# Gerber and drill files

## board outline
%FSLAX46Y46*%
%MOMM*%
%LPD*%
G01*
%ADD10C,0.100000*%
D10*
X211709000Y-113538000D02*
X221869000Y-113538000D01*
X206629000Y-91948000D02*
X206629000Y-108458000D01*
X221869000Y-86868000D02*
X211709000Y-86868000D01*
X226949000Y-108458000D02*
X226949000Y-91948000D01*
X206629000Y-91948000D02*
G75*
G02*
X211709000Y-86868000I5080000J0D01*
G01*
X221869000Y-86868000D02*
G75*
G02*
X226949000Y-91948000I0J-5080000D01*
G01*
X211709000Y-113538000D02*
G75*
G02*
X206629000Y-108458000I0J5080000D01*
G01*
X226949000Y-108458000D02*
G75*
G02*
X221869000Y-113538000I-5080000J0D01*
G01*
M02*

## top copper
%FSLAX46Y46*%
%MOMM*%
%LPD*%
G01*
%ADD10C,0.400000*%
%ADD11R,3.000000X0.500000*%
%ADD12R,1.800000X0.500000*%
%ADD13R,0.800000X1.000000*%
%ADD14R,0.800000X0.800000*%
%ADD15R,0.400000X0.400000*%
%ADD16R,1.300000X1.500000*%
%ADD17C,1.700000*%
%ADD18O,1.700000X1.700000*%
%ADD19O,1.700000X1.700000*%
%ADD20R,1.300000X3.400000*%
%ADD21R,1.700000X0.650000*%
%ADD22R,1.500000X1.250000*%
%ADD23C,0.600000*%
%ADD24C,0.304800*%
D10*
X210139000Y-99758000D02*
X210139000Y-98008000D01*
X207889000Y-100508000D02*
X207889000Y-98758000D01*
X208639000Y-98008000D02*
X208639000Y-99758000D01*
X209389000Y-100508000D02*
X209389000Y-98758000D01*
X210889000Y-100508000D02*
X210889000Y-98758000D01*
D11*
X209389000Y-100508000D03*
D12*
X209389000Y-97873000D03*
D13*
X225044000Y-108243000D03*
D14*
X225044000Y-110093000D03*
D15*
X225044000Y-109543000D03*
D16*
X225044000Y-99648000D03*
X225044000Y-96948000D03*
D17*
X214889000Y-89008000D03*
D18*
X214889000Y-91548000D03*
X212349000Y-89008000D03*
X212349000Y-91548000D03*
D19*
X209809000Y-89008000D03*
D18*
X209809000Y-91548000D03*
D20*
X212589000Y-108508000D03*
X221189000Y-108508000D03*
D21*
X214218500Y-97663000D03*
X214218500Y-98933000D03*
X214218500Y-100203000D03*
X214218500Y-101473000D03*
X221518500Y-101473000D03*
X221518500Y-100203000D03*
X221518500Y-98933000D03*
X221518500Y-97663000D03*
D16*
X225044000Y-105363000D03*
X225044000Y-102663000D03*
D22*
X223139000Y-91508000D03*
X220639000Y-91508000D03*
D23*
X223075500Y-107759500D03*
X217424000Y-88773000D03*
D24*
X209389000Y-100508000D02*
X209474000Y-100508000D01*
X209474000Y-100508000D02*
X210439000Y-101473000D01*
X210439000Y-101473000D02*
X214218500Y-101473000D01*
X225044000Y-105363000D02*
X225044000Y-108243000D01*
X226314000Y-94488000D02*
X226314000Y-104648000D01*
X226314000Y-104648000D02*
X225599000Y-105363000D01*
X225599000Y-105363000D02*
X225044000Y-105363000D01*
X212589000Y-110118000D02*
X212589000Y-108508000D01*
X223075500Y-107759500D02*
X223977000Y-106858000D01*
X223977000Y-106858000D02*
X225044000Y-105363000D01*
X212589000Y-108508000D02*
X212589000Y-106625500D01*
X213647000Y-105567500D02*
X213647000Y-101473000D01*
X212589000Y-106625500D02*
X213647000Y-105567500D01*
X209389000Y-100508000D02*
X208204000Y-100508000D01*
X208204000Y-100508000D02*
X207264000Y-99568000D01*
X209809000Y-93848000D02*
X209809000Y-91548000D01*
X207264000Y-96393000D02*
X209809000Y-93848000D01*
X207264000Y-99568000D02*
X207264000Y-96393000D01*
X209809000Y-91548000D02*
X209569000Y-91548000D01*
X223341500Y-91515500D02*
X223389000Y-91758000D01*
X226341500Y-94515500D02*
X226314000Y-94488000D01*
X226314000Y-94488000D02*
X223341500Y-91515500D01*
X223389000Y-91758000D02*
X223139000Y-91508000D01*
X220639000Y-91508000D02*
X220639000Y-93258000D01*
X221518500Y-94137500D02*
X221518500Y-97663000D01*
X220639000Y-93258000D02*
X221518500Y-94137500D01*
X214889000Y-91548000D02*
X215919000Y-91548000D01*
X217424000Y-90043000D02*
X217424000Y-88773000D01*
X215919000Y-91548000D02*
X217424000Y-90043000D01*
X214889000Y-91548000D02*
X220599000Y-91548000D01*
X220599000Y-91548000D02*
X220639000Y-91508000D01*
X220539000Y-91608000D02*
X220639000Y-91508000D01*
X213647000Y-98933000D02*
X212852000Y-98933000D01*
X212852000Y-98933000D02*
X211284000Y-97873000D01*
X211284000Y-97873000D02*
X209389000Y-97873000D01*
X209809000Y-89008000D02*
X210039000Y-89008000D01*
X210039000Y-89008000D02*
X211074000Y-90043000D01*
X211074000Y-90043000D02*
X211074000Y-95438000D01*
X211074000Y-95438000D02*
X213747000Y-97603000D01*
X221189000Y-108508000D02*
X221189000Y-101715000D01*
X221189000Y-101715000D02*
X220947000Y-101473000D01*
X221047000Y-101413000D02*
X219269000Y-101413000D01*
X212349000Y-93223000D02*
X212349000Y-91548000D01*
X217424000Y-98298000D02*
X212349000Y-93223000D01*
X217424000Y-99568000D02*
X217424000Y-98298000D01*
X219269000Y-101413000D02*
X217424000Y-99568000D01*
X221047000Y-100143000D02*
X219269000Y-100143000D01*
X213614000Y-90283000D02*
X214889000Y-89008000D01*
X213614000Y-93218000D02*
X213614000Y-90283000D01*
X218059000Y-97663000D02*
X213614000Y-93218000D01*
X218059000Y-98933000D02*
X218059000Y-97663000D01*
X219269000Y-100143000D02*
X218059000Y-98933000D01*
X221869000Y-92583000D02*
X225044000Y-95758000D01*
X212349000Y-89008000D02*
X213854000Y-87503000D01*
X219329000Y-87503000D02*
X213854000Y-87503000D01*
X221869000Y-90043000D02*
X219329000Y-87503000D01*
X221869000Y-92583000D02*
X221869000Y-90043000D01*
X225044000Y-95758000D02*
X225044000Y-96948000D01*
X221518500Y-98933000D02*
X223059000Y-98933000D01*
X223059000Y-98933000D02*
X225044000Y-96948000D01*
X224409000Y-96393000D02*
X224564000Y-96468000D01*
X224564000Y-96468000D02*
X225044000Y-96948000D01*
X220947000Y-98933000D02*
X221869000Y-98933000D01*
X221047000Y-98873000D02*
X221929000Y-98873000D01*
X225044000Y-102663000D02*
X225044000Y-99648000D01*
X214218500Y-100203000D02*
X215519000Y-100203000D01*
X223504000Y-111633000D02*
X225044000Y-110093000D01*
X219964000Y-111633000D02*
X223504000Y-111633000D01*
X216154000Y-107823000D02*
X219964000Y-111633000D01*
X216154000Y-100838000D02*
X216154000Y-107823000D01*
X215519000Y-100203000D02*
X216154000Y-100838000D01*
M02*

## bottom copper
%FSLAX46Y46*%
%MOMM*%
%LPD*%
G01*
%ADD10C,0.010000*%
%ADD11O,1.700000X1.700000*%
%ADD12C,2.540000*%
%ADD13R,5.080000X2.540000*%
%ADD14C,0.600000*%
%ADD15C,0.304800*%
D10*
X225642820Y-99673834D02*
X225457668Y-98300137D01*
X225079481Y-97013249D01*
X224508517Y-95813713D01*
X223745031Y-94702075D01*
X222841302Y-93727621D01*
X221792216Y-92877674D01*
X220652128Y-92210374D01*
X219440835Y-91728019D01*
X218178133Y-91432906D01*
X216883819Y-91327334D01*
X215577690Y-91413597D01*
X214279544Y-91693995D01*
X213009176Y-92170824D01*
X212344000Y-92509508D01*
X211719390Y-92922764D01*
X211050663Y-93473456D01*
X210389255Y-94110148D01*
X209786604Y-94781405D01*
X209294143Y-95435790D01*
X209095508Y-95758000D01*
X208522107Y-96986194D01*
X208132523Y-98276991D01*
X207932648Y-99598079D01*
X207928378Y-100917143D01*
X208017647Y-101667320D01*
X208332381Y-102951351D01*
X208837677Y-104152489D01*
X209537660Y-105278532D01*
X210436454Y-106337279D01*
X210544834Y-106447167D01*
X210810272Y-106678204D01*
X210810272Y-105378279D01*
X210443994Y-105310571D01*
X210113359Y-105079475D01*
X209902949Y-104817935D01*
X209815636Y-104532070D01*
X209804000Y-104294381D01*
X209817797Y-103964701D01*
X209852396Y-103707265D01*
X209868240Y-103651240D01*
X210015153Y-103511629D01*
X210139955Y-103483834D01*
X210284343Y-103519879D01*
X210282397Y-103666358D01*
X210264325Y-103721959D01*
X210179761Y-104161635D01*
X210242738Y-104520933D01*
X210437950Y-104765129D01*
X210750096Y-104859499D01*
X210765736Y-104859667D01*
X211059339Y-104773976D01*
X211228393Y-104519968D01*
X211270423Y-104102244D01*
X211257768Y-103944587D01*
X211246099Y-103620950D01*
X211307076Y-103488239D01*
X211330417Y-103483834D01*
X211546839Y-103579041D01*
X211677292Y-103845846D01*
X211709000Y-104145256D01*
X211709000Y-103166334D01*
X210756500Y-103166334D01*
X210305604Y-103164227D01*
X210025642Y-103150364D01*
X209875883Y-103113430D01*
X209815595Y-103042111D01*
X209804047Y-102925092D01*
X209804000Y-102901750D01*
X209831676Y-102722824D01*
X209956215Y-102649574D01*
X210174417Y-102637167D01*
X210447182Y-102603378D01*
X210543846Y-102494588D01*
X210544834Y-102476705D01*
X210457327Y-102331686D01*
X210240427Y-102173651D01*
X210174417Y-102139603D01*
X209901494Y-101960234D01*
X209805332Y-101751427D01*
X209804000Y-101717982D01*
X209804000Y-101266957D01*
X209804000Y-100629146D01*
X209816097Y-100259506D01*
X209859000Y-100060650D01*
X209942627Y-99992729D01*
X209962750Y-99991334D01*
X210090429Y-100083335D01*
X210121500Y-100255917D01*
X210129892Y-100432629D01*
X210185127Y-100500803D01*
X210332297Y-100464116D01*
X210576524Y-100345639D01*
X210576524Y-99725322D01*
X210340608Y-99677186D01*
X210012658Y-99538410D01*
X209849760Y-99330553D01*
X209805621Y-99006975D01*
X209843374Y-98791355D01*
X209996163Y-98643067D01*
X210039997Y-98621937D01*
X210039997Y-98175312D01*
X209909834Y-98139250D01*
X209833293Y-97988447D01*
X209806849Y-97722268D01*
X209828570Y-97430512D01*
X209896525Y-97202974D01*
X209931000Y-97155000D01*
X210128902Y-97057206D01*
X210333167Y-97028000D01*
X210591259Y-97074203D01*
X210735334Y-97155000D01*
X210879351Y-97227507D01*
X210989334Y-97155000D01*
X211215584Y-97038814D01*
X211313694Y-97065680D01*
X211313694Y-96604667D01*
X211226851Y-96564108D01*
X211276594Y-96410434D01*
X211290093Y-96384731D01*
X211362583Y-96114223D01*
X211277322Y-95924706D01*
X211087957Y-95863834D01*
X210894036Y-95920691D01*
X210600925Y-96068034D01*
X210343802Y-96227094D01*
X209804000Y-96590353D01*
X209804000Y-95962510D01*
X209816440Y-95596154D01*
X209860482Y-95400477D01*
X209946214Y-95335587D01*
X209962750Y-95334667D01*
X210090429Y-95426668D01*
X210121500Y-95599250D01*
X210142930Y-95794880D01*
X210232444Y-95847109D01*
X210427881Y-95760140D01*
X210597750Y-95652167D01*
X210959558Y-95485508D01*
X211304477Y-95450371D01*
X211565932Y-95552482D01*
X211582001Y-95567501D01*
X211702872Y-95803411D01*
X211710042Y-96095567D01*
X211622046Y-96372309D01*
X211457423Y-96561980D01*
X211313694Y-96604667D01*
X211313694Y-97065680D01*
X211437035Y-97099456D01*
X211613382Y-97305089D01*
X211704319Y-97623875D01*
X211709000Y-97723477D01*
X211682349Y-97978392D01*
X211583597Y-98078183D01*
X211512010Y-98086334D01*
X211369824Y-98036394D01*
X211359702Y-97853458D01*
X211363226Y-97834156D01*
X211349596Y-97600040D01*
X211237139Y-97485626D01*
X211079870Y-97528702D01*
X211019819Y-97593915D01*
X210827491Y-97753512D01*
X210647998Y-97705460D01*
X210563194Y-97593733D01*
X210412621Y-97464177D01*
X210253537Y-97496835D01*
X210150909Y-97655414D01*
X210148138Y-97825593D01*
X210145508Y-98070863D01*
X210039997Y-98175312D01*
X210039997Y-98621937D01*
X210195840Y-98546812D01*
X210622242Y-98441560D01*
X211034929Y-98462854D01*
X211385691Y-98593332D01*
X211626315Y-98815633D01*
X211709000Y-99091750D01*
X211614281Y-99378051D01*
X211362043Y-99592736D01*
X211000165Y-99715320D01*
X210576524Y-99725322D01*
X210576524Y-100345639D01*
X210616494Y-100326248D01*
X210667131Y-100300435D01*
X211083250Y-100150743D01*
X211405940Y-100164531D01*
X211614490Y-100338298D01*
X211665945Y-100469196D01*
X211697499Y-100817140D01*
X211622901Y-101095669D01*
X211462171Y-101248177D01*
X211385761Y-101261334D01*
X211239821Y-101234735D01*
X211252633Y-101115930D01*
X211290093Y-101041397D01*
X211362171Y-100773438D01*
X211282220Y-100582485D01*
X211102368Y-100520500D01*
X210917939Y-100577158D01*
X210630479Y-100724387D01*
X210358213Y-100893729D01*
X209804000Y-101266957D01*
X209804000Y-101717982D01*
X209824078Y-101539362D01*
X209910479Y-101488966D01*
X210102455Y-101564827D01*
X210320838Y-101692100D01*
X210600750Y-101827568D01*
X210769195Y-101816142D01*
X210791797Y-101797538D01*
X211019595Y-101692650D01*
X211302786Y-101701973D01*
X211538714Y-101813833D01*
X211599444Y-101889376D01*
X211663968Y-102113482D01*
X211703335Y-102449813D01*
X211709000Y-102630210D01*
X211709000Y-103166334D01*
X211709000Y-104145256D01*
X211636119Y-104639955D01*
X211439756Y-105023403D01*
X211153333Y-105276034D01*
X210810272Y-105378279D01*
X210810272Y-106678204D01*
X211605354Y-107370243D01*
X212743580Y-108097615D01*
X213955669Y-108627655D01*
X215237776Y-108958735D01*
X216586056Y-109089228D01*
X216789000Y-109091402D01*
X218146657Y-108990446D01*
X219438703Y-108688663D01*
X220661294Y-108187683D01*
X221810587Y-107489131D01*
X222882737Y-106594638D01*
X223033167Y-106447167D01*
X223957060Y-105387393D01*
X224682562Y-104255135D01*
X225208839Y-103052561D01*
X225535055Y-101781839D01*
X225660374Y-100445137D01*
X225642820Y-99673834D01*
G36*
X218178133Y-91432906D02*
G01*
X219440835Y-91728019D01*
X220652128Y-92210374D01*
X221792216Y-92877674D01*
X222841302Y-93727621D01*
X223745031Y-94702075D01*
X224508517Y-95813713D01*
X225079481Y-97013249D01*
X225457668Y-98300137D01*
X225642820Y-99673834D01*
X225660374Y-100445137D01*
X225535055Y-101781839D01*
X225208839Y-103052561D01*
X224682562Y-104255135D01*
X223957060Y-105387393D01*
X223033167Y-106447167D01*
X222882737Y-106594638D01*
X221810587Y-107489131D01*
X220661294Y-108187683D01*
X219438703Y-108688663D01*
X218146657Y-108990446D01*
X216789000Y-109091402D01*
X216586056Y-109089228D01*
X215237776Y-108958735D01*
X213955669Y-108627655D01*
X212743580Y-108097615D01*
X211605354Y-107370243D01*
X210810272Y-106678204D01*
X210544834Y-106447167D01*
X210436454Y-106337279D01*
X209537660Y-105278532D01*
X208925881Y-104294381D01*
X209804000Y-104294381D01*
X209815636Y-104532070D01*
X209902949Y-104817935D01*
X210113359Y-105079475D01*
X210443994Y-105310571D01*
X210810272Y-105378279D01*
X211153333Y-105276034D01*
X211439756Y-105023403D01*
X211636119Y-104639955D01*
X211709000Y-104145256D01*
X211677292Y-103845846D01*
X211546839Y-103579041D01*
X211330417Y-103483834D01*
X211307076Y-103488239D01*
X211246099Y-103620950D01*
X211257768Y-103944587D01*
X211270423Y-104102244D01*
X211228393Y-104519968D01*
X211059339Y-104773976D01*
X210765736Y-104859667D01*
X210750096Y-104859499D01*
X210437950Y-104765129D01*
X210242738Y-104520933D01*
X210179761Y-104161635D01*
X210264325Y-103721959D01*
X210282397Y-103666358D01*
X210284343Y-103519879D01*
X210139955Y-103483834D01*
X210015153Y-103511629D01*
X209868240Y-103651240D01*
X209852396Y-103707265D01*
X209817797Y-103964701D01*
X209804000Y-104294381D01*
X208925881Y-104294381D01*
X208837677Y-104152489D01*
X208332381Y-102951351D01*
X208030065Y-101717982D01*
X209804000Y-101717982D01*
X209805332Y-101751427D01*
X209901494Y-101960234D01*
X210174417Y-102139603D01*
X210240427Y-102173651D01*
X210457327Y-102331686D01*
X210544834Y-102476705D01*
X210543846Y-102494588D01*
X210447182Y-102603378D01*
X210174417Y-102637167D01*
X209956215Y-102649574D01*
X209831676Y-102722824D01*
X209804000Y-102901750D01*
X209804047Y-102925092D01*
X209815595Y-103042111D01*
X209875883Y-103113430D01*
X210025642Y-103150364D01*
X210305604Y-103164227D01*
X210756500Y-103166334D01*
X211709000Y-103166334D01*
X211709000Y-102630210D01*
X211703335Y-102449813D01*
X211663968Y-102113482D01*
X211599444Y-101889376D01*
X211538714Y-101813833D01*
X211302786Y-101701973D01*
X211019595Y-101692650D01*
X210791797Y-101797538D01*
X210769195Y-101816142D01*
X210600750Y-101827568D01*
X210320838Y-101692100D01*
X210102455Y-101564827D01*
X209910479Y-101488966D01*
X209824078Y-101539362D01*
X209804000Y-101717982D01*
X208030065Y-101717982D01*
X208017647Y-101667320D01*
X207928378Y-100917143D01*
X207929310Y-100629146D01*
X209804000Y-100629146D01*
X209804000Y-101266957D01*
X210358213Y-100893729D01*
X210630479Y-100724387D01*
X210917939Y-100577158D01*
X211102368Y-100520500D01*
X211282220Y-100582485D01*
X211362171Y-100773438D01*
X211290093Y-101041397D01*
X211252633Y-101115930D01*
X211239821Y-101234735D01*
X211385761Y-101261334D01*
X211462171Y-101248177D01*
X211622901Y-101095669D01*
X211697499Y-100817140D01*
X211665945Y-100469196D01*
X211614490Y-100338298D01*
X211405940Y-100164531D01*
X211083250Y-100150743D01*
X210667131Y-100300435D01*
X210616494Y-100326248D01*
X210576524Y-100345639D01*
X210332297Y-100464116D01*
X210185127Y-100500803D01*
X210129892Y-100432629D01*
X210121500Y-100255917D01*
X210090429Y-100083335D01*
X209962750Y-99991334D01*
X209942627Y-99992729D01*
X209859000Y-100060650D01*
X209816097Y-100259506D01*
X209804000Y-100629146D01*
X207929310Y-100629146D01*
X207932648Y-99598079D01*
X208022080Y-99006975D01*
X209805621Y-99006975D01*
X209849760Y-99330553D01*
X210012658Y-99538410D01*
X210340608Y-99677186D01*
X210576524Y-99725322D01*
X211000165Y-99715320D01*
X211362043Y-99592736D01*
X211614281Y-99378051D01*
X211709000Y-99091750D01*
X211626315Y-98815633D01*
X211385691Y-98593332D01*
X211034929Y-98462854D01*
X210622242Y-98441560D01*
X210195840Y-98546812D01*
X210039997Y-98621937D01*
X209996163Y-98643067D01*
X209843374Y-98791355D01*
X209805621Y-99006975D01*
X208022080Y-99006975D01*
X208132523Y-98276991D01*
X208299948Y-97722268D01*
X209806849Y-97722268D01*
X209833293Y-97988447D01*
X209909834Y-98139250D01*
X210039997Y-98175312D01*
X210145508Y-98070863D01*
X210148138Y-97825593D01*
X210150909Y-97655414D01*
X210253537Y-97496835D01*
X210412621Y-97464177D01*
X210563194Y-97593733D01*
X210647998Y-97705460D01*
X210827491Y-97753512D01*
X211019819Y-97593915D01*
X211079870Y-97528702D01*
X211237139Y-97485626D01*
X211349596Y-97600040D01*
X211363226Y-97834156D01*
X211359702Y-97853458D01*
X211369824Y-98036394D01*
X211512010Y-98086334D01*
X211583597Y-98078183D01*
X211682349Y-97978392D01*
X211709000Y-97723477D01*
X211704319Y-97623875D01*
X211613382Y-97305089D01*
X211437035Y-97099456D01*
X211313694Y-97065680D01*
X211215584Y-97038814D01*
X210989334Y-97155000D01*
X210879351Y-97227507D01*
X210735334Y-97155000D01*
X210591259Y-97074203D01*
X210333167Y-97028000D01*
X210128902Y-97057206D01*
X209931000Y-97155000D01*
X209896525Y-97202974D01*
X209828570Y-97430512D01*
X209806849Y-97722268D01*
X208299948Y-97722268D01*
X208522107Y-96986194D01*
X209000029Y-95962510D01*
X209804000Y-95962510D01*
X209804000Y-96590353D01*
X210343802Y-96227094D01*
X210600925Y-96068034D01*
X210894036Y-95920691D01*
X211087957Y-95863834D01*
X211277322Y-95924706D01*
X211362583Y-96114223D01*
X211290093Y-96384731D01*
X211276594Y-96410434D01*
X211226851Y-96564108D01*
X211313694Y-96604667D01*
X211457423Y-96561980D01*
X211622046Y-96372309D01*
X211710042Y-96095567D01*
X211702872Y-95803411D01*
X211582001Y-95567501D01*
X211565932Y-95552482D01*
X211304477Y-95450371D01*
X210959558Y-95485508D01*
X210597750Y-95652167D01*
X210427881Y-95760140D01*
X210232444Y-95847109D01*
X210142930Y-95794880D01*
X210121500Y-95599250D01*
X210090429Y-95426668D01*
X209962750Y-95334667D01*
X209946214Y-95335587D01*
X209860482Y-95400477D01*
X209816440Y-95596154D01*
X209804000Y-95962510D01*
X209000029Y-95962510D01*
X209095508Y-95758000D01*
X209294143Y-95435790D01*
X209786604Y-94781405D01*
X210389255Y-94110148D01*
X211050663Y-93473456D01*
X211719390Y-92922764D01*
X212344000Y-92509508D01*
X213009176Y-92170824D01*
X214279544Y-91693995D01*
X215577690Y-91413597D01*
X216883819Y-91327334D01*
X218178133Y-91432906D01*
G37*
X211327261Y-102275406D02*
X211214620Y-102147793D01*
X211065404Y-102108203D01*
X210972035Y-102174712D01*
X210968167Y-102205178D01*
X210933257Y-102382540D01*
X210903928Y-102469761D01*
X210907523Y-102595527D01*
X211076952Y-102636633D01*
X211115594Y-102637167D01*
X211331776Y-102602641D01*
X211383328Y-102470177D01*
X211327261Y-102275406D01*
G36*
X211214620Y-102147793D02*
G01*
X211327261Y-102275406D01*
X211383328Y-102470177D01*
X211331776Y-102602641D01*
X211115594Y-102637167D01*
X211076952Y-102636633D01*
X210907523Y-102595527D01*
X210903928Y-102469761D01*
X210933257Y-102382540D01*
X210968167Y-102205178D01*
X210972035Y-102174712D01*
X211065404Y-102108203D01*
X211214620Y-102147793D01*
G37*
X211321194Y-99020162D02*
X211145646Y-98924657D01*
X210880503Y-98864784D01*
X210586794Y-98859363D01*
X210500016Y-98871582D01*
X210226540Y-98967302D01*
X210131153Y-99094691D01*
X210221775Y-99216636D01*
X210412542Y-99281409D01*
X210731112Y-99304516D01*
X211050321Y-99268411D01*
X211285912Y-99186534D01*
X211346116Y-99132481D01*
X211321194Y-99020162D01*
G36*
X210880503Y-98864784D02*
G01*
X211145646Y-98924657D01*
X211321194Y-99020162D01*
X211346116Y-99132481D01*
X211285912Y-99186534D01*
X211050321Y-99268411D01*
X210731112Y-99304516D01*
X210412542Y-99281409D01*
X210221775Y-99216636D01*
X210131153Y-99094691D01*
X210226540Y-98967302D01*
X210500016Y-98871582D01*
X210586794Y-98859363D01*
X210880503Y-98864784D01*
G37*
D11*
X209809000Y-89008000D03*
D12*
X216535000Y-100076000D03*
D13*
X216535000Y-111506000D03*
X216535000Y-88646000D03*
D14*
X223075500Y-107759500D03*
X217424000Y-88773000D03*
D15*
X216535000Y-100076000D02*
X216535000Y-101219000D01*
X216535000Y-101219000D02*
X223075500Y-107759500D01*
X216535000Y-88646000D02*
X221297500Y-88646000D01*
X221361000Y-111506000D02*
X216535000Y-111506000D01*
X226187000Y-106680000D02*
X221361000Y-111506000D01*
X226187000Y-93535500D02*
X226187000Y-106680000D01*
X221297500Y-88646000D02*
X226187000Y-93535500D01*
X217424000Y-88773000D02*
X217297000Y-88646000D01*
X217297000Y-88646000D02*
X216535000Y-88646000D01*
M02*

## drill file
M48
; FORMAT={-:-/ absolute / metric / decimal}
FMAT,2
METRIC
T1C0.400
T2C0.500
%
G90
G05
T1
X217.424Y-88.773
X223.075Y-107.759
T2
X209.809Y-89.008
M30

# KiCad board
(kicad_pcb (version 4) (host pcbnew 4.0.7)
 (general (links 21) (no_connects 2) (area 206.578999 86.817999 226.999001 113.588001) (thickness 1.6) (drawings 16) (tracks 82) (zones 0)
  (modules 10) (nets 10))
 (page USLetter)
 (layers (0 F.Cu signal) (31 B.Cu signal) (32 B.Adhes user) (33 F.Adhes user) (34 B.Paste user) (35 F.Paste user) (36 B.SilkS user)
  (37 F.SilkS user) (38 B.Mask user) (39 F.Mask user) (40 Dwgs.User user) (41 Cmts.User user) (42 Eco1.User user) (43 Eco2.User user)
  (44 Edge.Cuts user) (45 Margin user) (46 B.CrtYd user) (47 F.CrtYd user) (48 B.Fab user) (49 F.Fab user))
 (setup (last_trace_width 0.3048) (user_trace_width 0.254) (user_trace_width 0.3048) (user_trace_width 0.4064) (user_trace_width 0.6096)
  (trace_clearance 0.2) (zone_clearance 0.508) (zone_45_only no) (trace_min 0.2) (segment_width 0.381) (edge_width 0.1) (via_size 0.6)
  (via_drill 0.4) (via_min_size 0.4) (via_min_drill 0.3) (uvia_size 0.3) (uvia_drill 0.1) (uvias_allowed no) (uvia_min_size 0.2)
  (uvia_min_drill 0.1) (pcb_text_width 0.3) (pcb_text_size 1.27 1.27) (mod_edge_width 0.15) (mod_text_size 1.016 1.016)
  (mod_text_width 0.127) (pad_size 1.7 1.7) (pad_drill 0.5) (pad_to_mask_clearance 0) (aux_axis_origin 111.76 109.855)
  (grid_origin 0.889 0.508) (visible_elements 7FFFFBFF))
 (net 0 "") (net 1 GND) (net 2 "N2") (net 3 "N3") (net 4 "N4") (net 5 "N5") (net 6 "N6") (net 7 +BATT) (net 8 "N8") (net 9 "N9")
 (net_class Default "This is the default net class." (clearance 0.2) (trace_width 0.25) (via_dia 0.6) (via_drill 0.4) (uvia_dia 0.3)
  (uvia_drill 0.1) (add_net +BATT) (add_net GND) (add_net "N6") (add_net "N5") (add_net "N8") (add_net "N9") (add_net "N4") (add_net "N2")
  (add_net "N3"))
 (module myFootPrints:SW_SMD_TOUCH (layer F.Cu) (at 209.389 98.508 180)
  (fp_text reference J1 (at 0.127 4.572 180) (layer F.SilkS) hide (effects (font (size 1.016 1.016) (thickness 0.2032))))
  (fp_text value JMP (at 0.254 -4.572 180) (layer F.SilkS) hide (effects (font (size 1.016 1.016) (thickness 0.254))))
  (fp_line (start -0.75 -1.25) (end -0.75 0.5) (layer F.Cu) (width 0.4))
  (fp_line (start 1.5 -2) (end 1.5 -0.25) (layer F.Cu) (width 0.4))
  (fp_line (start 0.75 0.5) (end 0.75 -1.25) (layer F.Cu) (width 0.4))
  (fp_line (start 0 -2) (end 0 -0.25) (layer F.Cu) (width 0.4))
  (fp_line (start -1.5 -2) (end -1.5 -0.25) (layer F.Cu) (width 0.4))
  (pad 1 smd rect (at 0 -2 180) (size 3 0.5) (layers F.Cu F.Paste F.Mask) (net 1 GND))
  (pad 2 smd rect (at 0 0.635 180) (size 1.8 0.5) (layers F.Cu F.Paste F.Mask) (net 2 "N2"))
  (pad 3 smd circle (at 0 -0.75 180) (size 3.5 3.5) (layers F.Paste F.Mask)))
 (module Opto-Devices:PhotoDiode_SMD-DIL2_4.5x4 (layer F.Cu) (at 225.044 109.093 90)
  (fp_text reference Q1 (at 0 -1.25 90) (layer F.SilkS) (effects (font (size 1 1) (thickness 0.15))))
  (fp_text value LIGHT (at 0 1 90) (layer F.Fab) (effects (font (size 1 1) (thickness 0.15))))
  (pad 2 smd rect (at 0.85 0 270) (size 1 0.8) (layers F.Cu F.Paste F.Mask) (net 1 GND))
  (pad 1 smd rect (at -1 0 270) (size 0.8 0.8) (layers F.Cu F.Paste F.Mask) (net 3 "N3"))
  (pad 1 smd rect (at -0.45 0 270) (size 0.4 0.4) (layers F.Cu F.Paste F.Mask) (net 3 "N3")))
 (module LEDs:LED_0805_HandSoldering (layer F.Cu) (at 225.044 98.298 90)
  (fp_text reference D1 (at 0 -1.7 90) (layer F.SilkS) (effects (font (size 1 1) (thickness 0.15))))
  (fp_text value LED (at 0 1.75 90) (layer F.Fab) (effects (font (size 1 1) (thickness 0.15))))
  (pad 1 smd rect (at -1.35 0 90) (size 1.5 1.3) (layers F.Cu F.Paste F.Mask) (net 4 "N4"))
  (pad 2 smd rect (at 1.35 0 90) (size 1.5 1.3) (layers F.Cu F.Paste F.Mask) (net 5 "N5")))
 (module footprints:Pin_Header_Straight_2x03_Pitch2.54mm (layer F.Cu) (at 214.889 89.008 270)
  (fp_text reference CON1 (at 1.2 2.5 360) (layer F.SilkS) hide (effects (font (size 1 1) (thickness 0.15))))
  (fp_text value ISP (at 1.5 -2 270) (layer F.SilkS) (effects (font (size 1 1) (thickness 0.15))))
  (pad 1 smd circle (at 0 0 270) (size 1.7 1.7) (layers F.Cu F.Paste F.Mask) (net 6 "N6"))
  (pad 2 smd oval (at 2.54 0 270) (size 1.7 1.7) (layers F.Cu F.Paste F.Mask) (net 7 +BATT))
  (pad 3 smd oval (at 0 2.54 270) (size 1.7 1.7) (layers F.Cu F.Paste F.Mask) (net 5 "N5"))
  (pad 4 smd oval (at 2.54 2.54 270) (size 1.7 1.7) (layers F.Cu F.Paste F.Mask) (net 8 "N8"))
  (pad 5 thru_hole oval (at 0 5.08 270) (size 1.7 1.7) (drill 0.5) (layers *.Cu F.Mask) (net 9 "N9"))
  (pad 6 smd oval (at 2.54 5.08 270) (size 1.7 1.7) (layers F.Cu F.Paste F.Mask) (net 1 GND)))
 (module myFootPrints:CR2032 (layer B.Cu) (at 216.789 100.203 90)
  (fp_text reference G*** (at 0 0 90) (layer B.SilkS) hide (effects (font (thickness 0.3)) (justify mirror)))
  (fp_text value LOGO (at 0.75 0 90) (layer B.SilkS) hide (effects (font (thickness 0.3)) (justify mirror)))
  (fp_poly
   (pts (xy 0.529166 8.85382) (xy 1.902863 8.668668) (xy 3.189751 8.290481) (xy 4.389287 7.719517) (xy 5.500925 6.956031)
    (xy 6.475379 6.052302) (xy 7.325326 5.003216) (xy 7.992626 3.863128) (xy 8.474981 2.651835) (xy 8.770094 1.389133)
    (xy 8.875666 0.094819) (xy 8.789403 -1.21131) (xy 8.509005 -2.509456) (xy 8.032176 -3.779824) (xy 7.693492 -4.445)
    (xy 7.280236 -5.06961) (xy 6.729544 -5.738337) (xy 6.092852 -6.399745) (xy 5.421595 -7.002396) (xy 4.76721 -7.494857)
    (xy 4.445 -7.693492) (xy 3.216806 -8.266893) (xy 1.926009 -8.656477) (xy 0.604921 -8.856352) (xy -0.714143 -8.860622)
    (xy -1.46432 -8.771353) (xy -2.748351 -8.456619) (xy -3.949489 -7.951323) (xy -5.075532 -7.25134) (xy -6.134279 -6.352546)
    (xy -6.244167 -6.244166) (xy -6.475204 -5.978728) (xy -5.175279 -5.978728) (xy -5.107571 -6.345006) (xy -4.876475 -6.675641)
    (xy -4.614935 -6.886051) (xy -4.32907 -6.973364) (xy -4.091381 -6.985) (xy -3.761701 -6.971203) (xy -3.504265 -6.936604)
    (xy -3.44824 -6.92076) (xy -3.308629 -6.773847) (xy -3.280834 -6.649045) (xy -3.316879 -6.504657) (xy -3.463358 -6.506603)
    (xy -3.518959 -6.524675) (xy -3.958635 -6.609239) (xy -4.317933 -6.546262) (xy -4.562129 -6.35105) (xy -4.656499 -6.038904)
    (xy -4.656667 -6.023264) (xy -4.570976 -5.729661) (xy -4.316968 -5.560607) (xy -3.899244 -5.518577) (xy -3.741587 -5.531232)
    (xy -3.41795 -5.542901) (xy -3.285239 -5.481924) (xy -3.280834 -5.458583) (xy -3.376041 -5.242161) (xy -3.642846 -5.111708)
    (xy -3.942256 -5.08) (xy -2.963334 -5.08) (xy -2.963334 -6.0325) (xy -2.961227 -6.483396) (xy -2.947364 -6.763358)
    (xy -2.91043 -6.913117) (xy -2.839111 -6.973405) (xy -2.722092 -6.984953) (xy -2.69875 -6.985) (xy -2.519824 -6.957324)
    (xy -2.446574 -6.832785) (xy -2.434167 -6.614583) (xy -2.400378 -6.341818) (xy -2.291588 -6.245154) (xy -2.273705 -6.244166)
    (xy -2.128686 -6.331673) (xy -1.970651 -6.548573) (xy -1.936603 -6.614583) (xy -1.757234 -6.887506) (xy -1.548427 -6.983668)
    (xy -1.514982 -6.985) (xy -1.063957 -6.985) (xy -0.426146 -6.985) (xy -0.056506 -6.972903) (xy 0.14235 -6.93) (xy 0.210271 -6.846373)
    (xy 0.211666 -6.82625) (xy 0.119665 -6.698571) (xy -0.052917 -6.6675) (xy -0.229629 -6.659108) (xy -0.297803 -6.603873)
    (xy -0.261116 -6.456703) (xy -0.142639 -6.212476) (xy 0.477678 -6.212476) (xy 0.525814 -6.448392) (xy 0.66459 -6.776342)
    (xy 0.872447 -6.93924) (xy 1.196025 -6.983379) (xy 1.411645 -6.945626) (xy 1.559933 -6.792837) (xy 1.581063 -6.749003)
    (xy 2.027688 -6.749003) (xy 2.06375 -6.879166) (xy 2.214553 -6.955707) (xy 2.480732 -6.982151) (xy 2.772488 -6.96043)
    (xy 3.000026 -6.892475) (xy 3.048 -6.858) (xy 3.145794 -6.660098) (xy 3.175 -6.455833) (xy 3.128797 -6.197741) (xy 3.048 -6.053666)
    (xy 2.975493 -5.909649) (xy 3.048 -5.799666) (xy 3.164186 -5.573416) (xy 3.13732 -5.475306) (xy 3.598333 -5.475306)
    (xy 3.638892 -5.562149) (xy 3.792566 -5.512406) (xy 3.818269 -5.498907) (xy 4.088777 -5.426417) (xy 4.278294 -5.511678)
    (xy 4.339166 -5.701043) (xy 4.282309 -5.894964) (xy 4.134966 -6.188075) (xy 3.975906 -6.445198) (xy 3.612647 -6.985) (xy 4.24049 -6.985)
    (xy 4.606846 -6.97256) (xy 4.802523 -6.928518) (xy 4.867413 -6.842786) (xy 4.868333 -6.82625) (xy 4.776332 -6.698571)
    (xy 4.60375 -6.6675) (xy 4.40812 -6.64607) (xy 4.355891 -6.556556) (xy 4.44286 -6.361119) (xy 4.550833 -6.19125) (xy 4.717492 -5.829442)
    (xy 4.752629 -5.484523) (xy 4.650518 -5.223068) (xy 4.635499 -5.206999) (xy 4.399589 -5.086128) (xy 4.107433 -5.078958)
    (xy 3.830691 -5.166954) (xy 3.64102 -5.331577) (xy 3.598333 -5.475306) (xy 3.13732 -5.475306) (xy 3.103544 -5.351965)
    (xy 2.897911 -5.175618) (xy 2.579125 -5.084681) (xy 2.479523 -5.08) (xy 2.224608 -5.106651) (xy 2.124817 -5.205403)
    (xy 2.116666 -5.27699) (xy 2.166606 -5.419176) (xy 2.349542 -5.429298) (xy 2.368844 -5.425774) (xy 2.60296 -5.439404)
    (xy 2.717374 -5.551861) (xy 2.674298 -5.70913) (xy 2.609085 -5.769181) (xy 2.449488 -5.961509) (xy 2.49754 -6.141002)
    (xy 2.609267 -6.225806) (xy 2.738823 -6.376379) (xy 2.706165 -6.535463) (xy 2.547586 -6.638091) (xy 2.377407 -6.640862)
    (xy 2.132137 -6.643492) (xy 2.027688 -6.749003) (xy 1.581063 -6.749003) (xy 1.656188 -6.59316) (xy 1.76144 -6.166758)
    (xy 1.740146 -5.754071) (xy 1.609668 -5.403309) (xy 1.387367 -5.162685) (xy 1.11125 -5.08) (xy 0.824949 -5.174719)
    (xy 0.610264 -5.426957) (xy 0.48768 -5.788835) (xy 0.477678 -6.212476) (xy -0.142639 -6.212476) (xy -0.123248 -6.172506)
    (xy -0.097435 -6.121869) (xy 0.052257 -5.70575) (xy 0.038469 -5.38306) (xy -0.135298 -5.17451) (xy -0.266196 -5.123055)
    (xy -0.61414 -5.091501) (xy -0.892669 -5.166099) (xy -1.045177 -5.326829) (xy -1.058334 -5.403239) (xy -1.031735 -5.549179)
    (xy -0.91293 -5.536367) (xy -0.838397 -5.498907) (xy -0.570438 -5.426829) (xy -0.379485 -5.50678) (xy -0.3175 -5.686632)
    (xy -0.374158 -5.871061) (xy -0.521387 -6.158521) (xy -0.690729 -6.430787) (xy -1.063957 -6.985) (xy -1.514982 -6.985)
    (xy -1.336362 -6.964922) (xy -1.285966 -6.878521) (xy -1.361827 -6.686545) (xy -1.4891 -6.468162) (xy -1.624568 -6.18825)
    (xy -1.613142 -6.019805) (xy -1.594538 -5.997203) (xy -1.48965 -5.769405) (xy -1.498973 -5.486214) (xy -1.610833 -5.250286)
    (xy -1.686376 -5.189556) (xy -1.910482 -5.125032) (xy -2.246813 -5.085665) (xy -2.42721 -5.08) (xy -2.963334 -5.08) (xy -3.942256 -5.08)
    (xy -4.436955 -5.152881) (xy -4.820403 -5.349244) (xy -5.073034 -5.635667) (xy -5.175279 -5.978728) (xy -6.475204 -5.978728)
    (xy -7.167243 -5.183646) (xy -7.894615 -4.04542) (xy -8.424655 -2.833331) (xy -8.755735 -1.551224) (xy -8.886228 -0.202944)
    (xy -8.888402 0) (xy -8.787446 1.357657) (xy -8.485663 2.649703) (xy -7.984683 3.872294) (xy -7.286131 5.021587) (xy -6.391638 6.093737)
    (xy -6.244167 6.244167) (xy -5.184393 7.16806) (xy -4.052135 7.893562) (xy -2.849561 8.419839) (xy -1.578839 8.746055)
    (xy -0.242137 8.871374) (xy 0.529166 8.85382))
   (layer B.Cu) (width 0.01))
  (fp_poly
   (pts (xy -2.072406 -5.461739) (xy -1.944793 -5.57438) (xy -1.905203 -5.723596) (xy -1.971712 -5.816965) (xy -2.002178 -5.820833)
    (xy -2.17954 -5.855743) (xy -2.266761 -5.885072) (xy -2.392527 -5.881477) (xy -2.433633 -5.712048) (xy -2.434167 -5.673406)
    (xy -2.399641 -5.457224) (xy -2.267177 -5.405672) (xy -2.072406 -5.461739))
   (layer B.Cu) (width 0.01))
  (fp_poly
   (pts (xy 1.182838 -5.467806) (xy 1.278343 -5.643354) (xy 1.338216 -5.908497) (xy 1.343637 -6.202206) (xy 1.331418 -6.288984)
    (xy 1.235698 -6.56246) (xy 1.108309 -6.657847) (xy 0.986364 -6.567225) (xy 0.921591 -6.376458) (xy 0.898484 -6.057888)
    (xy 0.934589 -5.738679) (xy 1.016466 -5.503088) (xy 1.070519 -5.442884) (xy 1.182838 -5.467806))
   (layer B.Cu) (width 0.01))
  (pad 3 smd circle (at 0 0 90) (size 17.78 17.78) (layers B.Paste B.Mask)))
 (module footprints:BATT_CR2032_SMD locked (layer B.Cu) (at 216.535 100.076 90)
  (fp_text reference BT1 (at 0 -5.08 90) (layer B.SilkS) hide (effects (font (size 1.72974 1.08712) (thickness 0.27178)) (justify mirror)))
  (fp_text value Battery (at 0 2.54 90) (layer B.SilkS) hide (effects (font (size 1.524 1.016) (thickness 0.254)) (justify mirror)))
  (pad 2 smd circle (at 0 0 90) (size 2.54 2.54) (layers B.Cu B.Paste B.Mask) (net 1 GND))
  (pad 1 smd rect (at -11.43 0 90) (size 2.54 5.08) (layers B.Cu B.Paste B.Mask) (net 7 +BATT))
  (pad 1 smd rect (at 11.43 0 90) (size 2.54 5.08) (layers B.Cu B.Paste B.Mask) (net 7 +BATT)))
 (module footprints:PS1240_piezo (layer F.Cu) (at 216.889 108.508)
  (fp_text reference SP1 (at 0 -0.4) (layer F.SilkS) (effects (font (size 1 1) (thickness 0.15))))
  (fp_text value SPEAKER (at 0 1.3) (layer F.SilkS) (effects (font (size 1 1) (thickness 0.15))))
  (pad 1 smd rect (at -4.3 0) (size 1.3 3.4) (layers F.Cu F.Paste F.Mask) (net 1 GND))
  (pad 2 smd rect (at 4.3 0) (size 1.3 3.4) (layers F.Cu F.Paste F.Mask) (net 8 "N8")))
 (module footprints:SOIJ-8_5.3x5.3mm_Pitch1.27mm (layer F.Cu) (at 217.8685 99.568)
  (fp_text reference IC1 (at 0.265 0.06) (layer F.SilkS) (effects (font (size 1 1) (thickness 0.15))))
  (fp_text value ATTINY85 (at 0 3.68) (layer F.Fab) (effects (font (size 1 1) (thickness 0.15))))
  (pad 1 smd rect (at -3.65 -1.905) (size 1.7 0.65) (layers F.Cu F.Paste F.Mask) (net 9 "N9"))
  (pad 2 smd rect (at -3.65 -0.635) (size 1.7 0.65) (layers F.Cu F.Paste F.Mask) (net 2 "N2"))
  (pad 3 smd rect (at -3.65 0.635) (size 1.7 0.65) (layers F.Cu F.Paste F.Mask) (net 3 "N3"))
  (pad 4 smd rect (at -3.65 1.905) (size 1.7 0.65) (layers F.Cu F.Paste F.Mask) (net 1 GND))
  (pad 5 smd rect (at 3.65 1.905) (size 1.7 0.65) (layers F.Cu F.Paste F.Mask) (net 8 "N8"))
  (pad 6 smd rect (at 3.65 0.635) (size 1.7 0.65) (layers F.Cu F.Paste F.Mask) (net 6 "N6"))
  (pad 7 smd rect (at 3.65 -0.635) (size 1.7 0.65) (layers F.Cu F.Paste F.Mask) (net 5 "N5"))
  (pad 8 smd rect (at 3.65 -1.905) (size 1.7 0.65) (layers F.Cu F.Paste F.Mask) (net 7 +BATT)))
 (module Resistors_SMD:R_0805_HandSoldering (layer F.Cu) (at 225.044 104.013 90)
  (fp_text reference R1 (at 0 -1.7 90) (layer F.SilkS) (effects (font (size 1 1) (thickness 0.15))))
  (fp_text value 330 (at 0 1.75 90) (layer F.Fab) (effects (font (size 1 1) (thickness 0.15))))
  (pad 1 smd rect (at -1.35 0 90) (size 1.5 1.3) (layers F.Cu F.Paste F.Mask) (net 1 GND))
  (pad 2 smd rect (at 1.35 0 90) (size 1.5 1.3) (layers F.Cu F.Paste F.Mask) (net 4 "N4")))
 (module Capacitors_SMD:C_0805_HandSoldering (layer F.Cu) (at 221.889 91.508 180)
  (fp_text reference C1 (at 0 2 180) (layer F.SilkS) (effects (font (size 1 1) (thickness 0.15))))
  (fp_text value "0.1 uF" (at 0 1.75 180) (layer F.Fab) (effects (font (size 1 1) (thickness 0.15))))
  (pad 1 smd rect (at -1.25 0 180) (size 1.5 1.25) (layers F.Cu F.Paste F.Mask) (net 1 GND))
  (pad 2 smd rect (at 1.25 0 180) (size 1.5 1.25) (layers F.Cu F.Paste F.Mask) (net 7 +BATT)))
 (gr_line (start 211.709 113.538) (end 221.869 113.538) (angle 90) (layer Edge.Cuts) (width 0.1))
 (gr_line (start 206.629 91.948) (end 206.629 108.458) (angle 90) (layer Edge.Cuts) (width 0.1))
 (gr_line (start 221.869 86.868) (end 211.709 86.868) (angle 90) (layer Edge.Cuts) (width 0.1))
 (gr_line (start 226.949 108.458) (end 226.949 91.948) (angle 90) (layer Edge.Cuts) (width 0.1))
 (gr_arc (start 211.709 91.948) (end 206.629 91.948) (angle 90) (layer Edge.Cuts) (width 0.1))
 (gr_arc (start 221.869 91.948) (end 221.869 86.868) (angle 90) (layer Edge.Cuts) (width 0.1))
 (gr_arc (start 211.709 108.458) (end 211.709 113.538) (angle 90) (layer Edge.Cuts) (width 0.1))
 (gr_arc (start 221.869 108.458) (end 226.949 108.458) (angle 90) (layer Edge.Cuts) (width 0.1))
 (segment (start 209.389 100.508) (end 209.474 100.508) (width 0.3048) (layer F.Cu) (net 1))
 (segment (start 209.474 100.508) (end 210.439 101.473) (width 0.3048) (layer F.Cu) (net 1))
 (segment (start 210.439 101.473) (end 214.2185 101.473) (width 0.3048) (layer F.Cu) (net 1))
 (segment (start 225.044 105.363) (end 225.044 108.243) (width 0.3048) (layer F.Cu) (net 1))
 (segment (start 226.314 94.488) (end 226.314 104.648) (width 0.3048) (layer F.Cu) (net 1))
 (segment (start 226.314 104.648) (end 225.599 105.363) (width 0.3048) (layer F.Cu) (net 1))
 (segment (start 225.599 105.363) (end 225.044 105.363) (width 0.3048) (layer F.Cu) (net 1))
 (segment (start 212.589 110.118) (end 212.589 108.508) (width 0.3048) (layer F.Cu) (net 1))
 (segment (start 216.535 100.076) (end 216.535 101.219) (width 0.3048) (layer B.Cu) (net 1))
 (segment (start 216.535 101.219) (end 223.0755 107.7595) (width 0.3048) (layer B.Cu) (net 1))
 (via (at 223.0755 107.7595) (size 0.6) (drill 0.4) (layers F.Cu B.Cu) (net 1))
 (segment (start 223.0755 107.7595) (end 223.977 106.858) (width 0.3048) (layer F.Cu) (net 1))
 (segment (start 223.977 106.858) (end 225.044 105.363) (width 0.3048) (layer F.Cu) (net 1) (status 20))
 (segment (start 212.589 108.508) (end 212.589 106.6255) (width 0.3048) (layer F.Cu) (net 1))
 (segment (start 213.647 105.5675) (end 213.647 101.473) (width 0.3048) (layer F.Cu) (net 1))
 (segment (start 212.589 106.6255) (end 213.647 105.5675) (width 0.3048) (layer F.Cu) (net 1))
 (segment (start 209.389 100.508) (end 208.204 100.508) (width 0.3048) (layer F.Cu) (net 1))
 (segment (start 208.204 100.508) (end 207.264 99.568) (width 0.3048) (layer F.Cu) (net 1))
 (segment (start 209.809 93.848) (end 209.809 91.548) (width 0.3048) (layer F.Cu) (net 1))
 (segment (start 207.264 96.393) (end 209.809 93.848) (width 0.3048) (layer F.Cu) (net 1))
 (segment (start 207.264 99.568) (end 207.264 96.393) (width 0.3048) (layer F.Cu) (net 1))
 (segment (start 209.809 91.548) (end 209.569 91.548) (width 0.3048) (layer F.Cu) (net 1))
 (segment (start 223.3415 91.5155) (end 223.389 91.758) (width 0.3048) (layer F.Cu) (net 1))
 (segment (start 226.3415 94.5155) (end 226.314 94.488) (width 0.3048) (layer F.Cu) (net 1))
 (segment (start 226.314 94.488) (end 223.3415 91.5155) (width 0.3048) (layer F.Cu) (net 1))
 (segment (start 223.389 91.758) (end 223.139 91.508) (width 0.3048) (layer F.Cu) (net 1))
 (segment (start 220.639 91.508) (end 220.639 93.258) (width 0.3048) (layer F.Cu) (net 7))
 (segment (start 221.5185 94.1375) (end 221.5185 97.663) (width 0.3048) (layer F.Cu) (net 7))
 (segment (start 220.639 93.258) (end 221.5185 94.1375) (width 0.3048) (layer F.Cu) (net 7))
 (segment (start 216.535 88.646) (end 221.2975 88.646) (width 0.3048) (layer B.Cu) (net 7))
 (segment (start 221.361 111.506) (end 216.535 111.506) (width 0.3048) (layer B.Cu) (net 7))
 (segment (start 226.187 106.68) (end 221.361 111.506) (width 0.3048) (layer B.Cu) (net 7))
 (segment (start 226.187 93.5355) (end 226.187 106.68) (width 0.3048) (layer B.Cu) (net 7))
 (segment (start 221.2975 88.646) (end 226.187 93.5355) (width 0.3048) (layer B.Cu) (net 7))
 (segment (start 214.889 91.548) (end 215.919 91.548) (width 0.3048) (layer F.Cu) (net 7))
 (segment (start 217.424 88.773) (end 217.297 88.646) (width 0.3048) (layer B.Cu) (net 7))
 (via (at 217.424 88.773) (size 0.6) (drill 0.4) (layers F.Cu B.Cu) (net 7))
 (segment (start 217.424 90.043) (end 217.424 88.773) (width 0.3048) (layer F.Cu) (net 7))
 (segment (start 215.919 91.548) (end 217.424 90.043) (width 0.3048) (layer F.Cu) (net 7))
 (segment (start 217.297 88.646) (end 216.535 88.646) (width 0.3048) (layer B.Cu) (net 7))
 (segment (start 214.889 91.548) (end 220.599 91.548) (width 0.3048) (layer F.Cu) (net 7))
 (segment (start 220.599 91.548) (end 220.639 91.508) (width 0.3048) (layer F.Cu) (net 7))
 (segment (start 220.539 91.608) (end 220.639 91.508) (width 0.3048) (layer F.Cu) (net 7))
 (segment (start 213.647 98.933) (end 212.852 98.933) (width 0.3048) (layer F.Cu) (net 2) (status 30))
 (segment (start 212.852 98.933) (end 211.284 97.873) (width 0.3048) (layer F.Cu) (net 2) (status 10))
 (segment (start 211.284 97.873) (end 209.389 97.873) (width 0.3048) (layer F.Cu) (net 2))
 (segment (start 209.809 89.008) (end 210.039 89.008) (width 0.3048) (layer F.Cu) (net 9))
 (segment (start 210.039 89.008) (end 211.074 90.043) (width 0.3048) (layer F.Cu) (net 9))
 (segment (start 211.074 90.043) (end 211.074 95.438) (width 0.3048) (layer F.Cu) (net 9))
 (segment (start 211.074 95.438) (end 213.747 97.603) (width 0.3048) (layer F.Cu) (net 9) (status 20))
 (segment (start 221.189 108.508) (end 221.189 101.715) (width 0.3048) (layer F.Cu) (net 8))
 (segment (start 221.189 101.715) (end 220.947 101.473) (width 0.3048) (layer F.Cu) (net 8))
 (segment (start 221.047 101.413) (end 219.269 101.413) (width 0.3048) (layer F.Cu) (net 8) (status 10))
 (segment (start 212.349 93.223) (end 212.349 91.548) (width 0.3048) (layer F.Cu) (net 8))
 (segment (start 217.424 98.298) (end 212.349 93.223) (width 0.3048) (layer F.Cu) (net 8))
 (segment (start 217.424 99.568) (end 217.424 98.298) (width 0.3048) (layer F.Cu) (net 8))
 (segment (start 219.269 101.413) (end 217.424 99.568) (width 0.3048) (layer F.Cu) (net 8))
 (segment (start 221.047 100.143) (end 219.269 100.143) (width 0.3048) (layer F.Cu) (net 6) (status 10))
 (segment (start 213.614 90.283) (end 214.889 89.008) (width 0.3048) (layer F.Cu) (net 6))
 (segment (start 213.614 93.218) (end 213.614 90.283) (width 0.3048) (layer F.Cu) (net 6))
 (segment (start 218.059 97.663) (end 213.614 93.218) (width 0.3048) (layer F.Cu) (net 6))
 (segment (start 218.059 98.933) (end 218.059 97.663) (width 0.3048) (layer F.Cu) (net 6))
 (segment (start 219.269 100.143) (end 218.059 98.933) (width 0.3048) (layer F.Cu) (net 6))
 (segment (start 221.869 92.583) (end 225.044 95.758) (width 0.3048) (layer F.Cu) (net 5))
 (segment (start 212.349 89.008) (end 213.854 87.503) (width 0.3048) (layer F.Cu) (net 5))
 (segment (start 219.329 87.503) (end 213.854 87.503) (width 0.3048) (layer F.Cu) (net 5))
 (segment (start 221.869 90.043) (end 219.329 87.503) (width 0.3048) (layer F.Cu) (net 5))
 (segment (start 221.869 92.583) (end 221.869 90.043) (width 0.3048) (layer F.Cu) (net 5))
 (segment (start 225.044 95.758) (end 225.044 96.948) (width 0.3048) (layer F.Cu) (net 5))
 (segment (start 221.5185 98.933) (end 223.059 98.933) (width 0.3048) (layer F.Cu) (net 5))
 (segment (start 223.059 98.933) (end 225.044 96.948) (width 0.3048) (layer F.Cu) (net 5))
 (segment (start 224.409 96.393) (end 224.564 96.468) (width 0.3048) (layer F.Cu) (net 5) (status 20))
 (segment (start 224.564 96.468) (end 225.044 96.948) (width 0.3048) (layer F.Cu) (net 5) (status 30))
 (segment (start 220.947 98.933) (end 221.869 98.933) (width 0.3048) (layer F.Cu) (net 5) (status 10))
 (segment (start 221.047 98.873) (end 221.929 98.873) (width 0.3048) (layer F.Cu) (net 5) (status 10))
 (segment (start 225.044 102.663) (end 225.044 99.648) (width 0.3048) (layer F.Cu) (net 4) (status 10))
 (segment (start 214.2185 100.203) (end 215.519 100.203) (width 0.3048) (layer F.Cu) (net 3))
 (segment (start 223.504 111.633) (end 225.044 110.093) (width 0.3048) (layer F.Cu) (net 3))
 (segment (start 219.964 111.633) (end 223.504 111.633) (width 0.3048) (layer F.Cu) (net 3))
 (segment (start 216.154 107.823) (end 219.964 111.633) (width 0.3048) (layer F.Cu) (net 3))
 (segment (start 216.154 100.838) (end 216.154 107.823) (width 0.3048) (layer F.Cu) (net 3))
 (segment (start 215.519 100.203) (end 216.154 100.838) (width 0.3048) (layer F.Cu) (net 3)))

